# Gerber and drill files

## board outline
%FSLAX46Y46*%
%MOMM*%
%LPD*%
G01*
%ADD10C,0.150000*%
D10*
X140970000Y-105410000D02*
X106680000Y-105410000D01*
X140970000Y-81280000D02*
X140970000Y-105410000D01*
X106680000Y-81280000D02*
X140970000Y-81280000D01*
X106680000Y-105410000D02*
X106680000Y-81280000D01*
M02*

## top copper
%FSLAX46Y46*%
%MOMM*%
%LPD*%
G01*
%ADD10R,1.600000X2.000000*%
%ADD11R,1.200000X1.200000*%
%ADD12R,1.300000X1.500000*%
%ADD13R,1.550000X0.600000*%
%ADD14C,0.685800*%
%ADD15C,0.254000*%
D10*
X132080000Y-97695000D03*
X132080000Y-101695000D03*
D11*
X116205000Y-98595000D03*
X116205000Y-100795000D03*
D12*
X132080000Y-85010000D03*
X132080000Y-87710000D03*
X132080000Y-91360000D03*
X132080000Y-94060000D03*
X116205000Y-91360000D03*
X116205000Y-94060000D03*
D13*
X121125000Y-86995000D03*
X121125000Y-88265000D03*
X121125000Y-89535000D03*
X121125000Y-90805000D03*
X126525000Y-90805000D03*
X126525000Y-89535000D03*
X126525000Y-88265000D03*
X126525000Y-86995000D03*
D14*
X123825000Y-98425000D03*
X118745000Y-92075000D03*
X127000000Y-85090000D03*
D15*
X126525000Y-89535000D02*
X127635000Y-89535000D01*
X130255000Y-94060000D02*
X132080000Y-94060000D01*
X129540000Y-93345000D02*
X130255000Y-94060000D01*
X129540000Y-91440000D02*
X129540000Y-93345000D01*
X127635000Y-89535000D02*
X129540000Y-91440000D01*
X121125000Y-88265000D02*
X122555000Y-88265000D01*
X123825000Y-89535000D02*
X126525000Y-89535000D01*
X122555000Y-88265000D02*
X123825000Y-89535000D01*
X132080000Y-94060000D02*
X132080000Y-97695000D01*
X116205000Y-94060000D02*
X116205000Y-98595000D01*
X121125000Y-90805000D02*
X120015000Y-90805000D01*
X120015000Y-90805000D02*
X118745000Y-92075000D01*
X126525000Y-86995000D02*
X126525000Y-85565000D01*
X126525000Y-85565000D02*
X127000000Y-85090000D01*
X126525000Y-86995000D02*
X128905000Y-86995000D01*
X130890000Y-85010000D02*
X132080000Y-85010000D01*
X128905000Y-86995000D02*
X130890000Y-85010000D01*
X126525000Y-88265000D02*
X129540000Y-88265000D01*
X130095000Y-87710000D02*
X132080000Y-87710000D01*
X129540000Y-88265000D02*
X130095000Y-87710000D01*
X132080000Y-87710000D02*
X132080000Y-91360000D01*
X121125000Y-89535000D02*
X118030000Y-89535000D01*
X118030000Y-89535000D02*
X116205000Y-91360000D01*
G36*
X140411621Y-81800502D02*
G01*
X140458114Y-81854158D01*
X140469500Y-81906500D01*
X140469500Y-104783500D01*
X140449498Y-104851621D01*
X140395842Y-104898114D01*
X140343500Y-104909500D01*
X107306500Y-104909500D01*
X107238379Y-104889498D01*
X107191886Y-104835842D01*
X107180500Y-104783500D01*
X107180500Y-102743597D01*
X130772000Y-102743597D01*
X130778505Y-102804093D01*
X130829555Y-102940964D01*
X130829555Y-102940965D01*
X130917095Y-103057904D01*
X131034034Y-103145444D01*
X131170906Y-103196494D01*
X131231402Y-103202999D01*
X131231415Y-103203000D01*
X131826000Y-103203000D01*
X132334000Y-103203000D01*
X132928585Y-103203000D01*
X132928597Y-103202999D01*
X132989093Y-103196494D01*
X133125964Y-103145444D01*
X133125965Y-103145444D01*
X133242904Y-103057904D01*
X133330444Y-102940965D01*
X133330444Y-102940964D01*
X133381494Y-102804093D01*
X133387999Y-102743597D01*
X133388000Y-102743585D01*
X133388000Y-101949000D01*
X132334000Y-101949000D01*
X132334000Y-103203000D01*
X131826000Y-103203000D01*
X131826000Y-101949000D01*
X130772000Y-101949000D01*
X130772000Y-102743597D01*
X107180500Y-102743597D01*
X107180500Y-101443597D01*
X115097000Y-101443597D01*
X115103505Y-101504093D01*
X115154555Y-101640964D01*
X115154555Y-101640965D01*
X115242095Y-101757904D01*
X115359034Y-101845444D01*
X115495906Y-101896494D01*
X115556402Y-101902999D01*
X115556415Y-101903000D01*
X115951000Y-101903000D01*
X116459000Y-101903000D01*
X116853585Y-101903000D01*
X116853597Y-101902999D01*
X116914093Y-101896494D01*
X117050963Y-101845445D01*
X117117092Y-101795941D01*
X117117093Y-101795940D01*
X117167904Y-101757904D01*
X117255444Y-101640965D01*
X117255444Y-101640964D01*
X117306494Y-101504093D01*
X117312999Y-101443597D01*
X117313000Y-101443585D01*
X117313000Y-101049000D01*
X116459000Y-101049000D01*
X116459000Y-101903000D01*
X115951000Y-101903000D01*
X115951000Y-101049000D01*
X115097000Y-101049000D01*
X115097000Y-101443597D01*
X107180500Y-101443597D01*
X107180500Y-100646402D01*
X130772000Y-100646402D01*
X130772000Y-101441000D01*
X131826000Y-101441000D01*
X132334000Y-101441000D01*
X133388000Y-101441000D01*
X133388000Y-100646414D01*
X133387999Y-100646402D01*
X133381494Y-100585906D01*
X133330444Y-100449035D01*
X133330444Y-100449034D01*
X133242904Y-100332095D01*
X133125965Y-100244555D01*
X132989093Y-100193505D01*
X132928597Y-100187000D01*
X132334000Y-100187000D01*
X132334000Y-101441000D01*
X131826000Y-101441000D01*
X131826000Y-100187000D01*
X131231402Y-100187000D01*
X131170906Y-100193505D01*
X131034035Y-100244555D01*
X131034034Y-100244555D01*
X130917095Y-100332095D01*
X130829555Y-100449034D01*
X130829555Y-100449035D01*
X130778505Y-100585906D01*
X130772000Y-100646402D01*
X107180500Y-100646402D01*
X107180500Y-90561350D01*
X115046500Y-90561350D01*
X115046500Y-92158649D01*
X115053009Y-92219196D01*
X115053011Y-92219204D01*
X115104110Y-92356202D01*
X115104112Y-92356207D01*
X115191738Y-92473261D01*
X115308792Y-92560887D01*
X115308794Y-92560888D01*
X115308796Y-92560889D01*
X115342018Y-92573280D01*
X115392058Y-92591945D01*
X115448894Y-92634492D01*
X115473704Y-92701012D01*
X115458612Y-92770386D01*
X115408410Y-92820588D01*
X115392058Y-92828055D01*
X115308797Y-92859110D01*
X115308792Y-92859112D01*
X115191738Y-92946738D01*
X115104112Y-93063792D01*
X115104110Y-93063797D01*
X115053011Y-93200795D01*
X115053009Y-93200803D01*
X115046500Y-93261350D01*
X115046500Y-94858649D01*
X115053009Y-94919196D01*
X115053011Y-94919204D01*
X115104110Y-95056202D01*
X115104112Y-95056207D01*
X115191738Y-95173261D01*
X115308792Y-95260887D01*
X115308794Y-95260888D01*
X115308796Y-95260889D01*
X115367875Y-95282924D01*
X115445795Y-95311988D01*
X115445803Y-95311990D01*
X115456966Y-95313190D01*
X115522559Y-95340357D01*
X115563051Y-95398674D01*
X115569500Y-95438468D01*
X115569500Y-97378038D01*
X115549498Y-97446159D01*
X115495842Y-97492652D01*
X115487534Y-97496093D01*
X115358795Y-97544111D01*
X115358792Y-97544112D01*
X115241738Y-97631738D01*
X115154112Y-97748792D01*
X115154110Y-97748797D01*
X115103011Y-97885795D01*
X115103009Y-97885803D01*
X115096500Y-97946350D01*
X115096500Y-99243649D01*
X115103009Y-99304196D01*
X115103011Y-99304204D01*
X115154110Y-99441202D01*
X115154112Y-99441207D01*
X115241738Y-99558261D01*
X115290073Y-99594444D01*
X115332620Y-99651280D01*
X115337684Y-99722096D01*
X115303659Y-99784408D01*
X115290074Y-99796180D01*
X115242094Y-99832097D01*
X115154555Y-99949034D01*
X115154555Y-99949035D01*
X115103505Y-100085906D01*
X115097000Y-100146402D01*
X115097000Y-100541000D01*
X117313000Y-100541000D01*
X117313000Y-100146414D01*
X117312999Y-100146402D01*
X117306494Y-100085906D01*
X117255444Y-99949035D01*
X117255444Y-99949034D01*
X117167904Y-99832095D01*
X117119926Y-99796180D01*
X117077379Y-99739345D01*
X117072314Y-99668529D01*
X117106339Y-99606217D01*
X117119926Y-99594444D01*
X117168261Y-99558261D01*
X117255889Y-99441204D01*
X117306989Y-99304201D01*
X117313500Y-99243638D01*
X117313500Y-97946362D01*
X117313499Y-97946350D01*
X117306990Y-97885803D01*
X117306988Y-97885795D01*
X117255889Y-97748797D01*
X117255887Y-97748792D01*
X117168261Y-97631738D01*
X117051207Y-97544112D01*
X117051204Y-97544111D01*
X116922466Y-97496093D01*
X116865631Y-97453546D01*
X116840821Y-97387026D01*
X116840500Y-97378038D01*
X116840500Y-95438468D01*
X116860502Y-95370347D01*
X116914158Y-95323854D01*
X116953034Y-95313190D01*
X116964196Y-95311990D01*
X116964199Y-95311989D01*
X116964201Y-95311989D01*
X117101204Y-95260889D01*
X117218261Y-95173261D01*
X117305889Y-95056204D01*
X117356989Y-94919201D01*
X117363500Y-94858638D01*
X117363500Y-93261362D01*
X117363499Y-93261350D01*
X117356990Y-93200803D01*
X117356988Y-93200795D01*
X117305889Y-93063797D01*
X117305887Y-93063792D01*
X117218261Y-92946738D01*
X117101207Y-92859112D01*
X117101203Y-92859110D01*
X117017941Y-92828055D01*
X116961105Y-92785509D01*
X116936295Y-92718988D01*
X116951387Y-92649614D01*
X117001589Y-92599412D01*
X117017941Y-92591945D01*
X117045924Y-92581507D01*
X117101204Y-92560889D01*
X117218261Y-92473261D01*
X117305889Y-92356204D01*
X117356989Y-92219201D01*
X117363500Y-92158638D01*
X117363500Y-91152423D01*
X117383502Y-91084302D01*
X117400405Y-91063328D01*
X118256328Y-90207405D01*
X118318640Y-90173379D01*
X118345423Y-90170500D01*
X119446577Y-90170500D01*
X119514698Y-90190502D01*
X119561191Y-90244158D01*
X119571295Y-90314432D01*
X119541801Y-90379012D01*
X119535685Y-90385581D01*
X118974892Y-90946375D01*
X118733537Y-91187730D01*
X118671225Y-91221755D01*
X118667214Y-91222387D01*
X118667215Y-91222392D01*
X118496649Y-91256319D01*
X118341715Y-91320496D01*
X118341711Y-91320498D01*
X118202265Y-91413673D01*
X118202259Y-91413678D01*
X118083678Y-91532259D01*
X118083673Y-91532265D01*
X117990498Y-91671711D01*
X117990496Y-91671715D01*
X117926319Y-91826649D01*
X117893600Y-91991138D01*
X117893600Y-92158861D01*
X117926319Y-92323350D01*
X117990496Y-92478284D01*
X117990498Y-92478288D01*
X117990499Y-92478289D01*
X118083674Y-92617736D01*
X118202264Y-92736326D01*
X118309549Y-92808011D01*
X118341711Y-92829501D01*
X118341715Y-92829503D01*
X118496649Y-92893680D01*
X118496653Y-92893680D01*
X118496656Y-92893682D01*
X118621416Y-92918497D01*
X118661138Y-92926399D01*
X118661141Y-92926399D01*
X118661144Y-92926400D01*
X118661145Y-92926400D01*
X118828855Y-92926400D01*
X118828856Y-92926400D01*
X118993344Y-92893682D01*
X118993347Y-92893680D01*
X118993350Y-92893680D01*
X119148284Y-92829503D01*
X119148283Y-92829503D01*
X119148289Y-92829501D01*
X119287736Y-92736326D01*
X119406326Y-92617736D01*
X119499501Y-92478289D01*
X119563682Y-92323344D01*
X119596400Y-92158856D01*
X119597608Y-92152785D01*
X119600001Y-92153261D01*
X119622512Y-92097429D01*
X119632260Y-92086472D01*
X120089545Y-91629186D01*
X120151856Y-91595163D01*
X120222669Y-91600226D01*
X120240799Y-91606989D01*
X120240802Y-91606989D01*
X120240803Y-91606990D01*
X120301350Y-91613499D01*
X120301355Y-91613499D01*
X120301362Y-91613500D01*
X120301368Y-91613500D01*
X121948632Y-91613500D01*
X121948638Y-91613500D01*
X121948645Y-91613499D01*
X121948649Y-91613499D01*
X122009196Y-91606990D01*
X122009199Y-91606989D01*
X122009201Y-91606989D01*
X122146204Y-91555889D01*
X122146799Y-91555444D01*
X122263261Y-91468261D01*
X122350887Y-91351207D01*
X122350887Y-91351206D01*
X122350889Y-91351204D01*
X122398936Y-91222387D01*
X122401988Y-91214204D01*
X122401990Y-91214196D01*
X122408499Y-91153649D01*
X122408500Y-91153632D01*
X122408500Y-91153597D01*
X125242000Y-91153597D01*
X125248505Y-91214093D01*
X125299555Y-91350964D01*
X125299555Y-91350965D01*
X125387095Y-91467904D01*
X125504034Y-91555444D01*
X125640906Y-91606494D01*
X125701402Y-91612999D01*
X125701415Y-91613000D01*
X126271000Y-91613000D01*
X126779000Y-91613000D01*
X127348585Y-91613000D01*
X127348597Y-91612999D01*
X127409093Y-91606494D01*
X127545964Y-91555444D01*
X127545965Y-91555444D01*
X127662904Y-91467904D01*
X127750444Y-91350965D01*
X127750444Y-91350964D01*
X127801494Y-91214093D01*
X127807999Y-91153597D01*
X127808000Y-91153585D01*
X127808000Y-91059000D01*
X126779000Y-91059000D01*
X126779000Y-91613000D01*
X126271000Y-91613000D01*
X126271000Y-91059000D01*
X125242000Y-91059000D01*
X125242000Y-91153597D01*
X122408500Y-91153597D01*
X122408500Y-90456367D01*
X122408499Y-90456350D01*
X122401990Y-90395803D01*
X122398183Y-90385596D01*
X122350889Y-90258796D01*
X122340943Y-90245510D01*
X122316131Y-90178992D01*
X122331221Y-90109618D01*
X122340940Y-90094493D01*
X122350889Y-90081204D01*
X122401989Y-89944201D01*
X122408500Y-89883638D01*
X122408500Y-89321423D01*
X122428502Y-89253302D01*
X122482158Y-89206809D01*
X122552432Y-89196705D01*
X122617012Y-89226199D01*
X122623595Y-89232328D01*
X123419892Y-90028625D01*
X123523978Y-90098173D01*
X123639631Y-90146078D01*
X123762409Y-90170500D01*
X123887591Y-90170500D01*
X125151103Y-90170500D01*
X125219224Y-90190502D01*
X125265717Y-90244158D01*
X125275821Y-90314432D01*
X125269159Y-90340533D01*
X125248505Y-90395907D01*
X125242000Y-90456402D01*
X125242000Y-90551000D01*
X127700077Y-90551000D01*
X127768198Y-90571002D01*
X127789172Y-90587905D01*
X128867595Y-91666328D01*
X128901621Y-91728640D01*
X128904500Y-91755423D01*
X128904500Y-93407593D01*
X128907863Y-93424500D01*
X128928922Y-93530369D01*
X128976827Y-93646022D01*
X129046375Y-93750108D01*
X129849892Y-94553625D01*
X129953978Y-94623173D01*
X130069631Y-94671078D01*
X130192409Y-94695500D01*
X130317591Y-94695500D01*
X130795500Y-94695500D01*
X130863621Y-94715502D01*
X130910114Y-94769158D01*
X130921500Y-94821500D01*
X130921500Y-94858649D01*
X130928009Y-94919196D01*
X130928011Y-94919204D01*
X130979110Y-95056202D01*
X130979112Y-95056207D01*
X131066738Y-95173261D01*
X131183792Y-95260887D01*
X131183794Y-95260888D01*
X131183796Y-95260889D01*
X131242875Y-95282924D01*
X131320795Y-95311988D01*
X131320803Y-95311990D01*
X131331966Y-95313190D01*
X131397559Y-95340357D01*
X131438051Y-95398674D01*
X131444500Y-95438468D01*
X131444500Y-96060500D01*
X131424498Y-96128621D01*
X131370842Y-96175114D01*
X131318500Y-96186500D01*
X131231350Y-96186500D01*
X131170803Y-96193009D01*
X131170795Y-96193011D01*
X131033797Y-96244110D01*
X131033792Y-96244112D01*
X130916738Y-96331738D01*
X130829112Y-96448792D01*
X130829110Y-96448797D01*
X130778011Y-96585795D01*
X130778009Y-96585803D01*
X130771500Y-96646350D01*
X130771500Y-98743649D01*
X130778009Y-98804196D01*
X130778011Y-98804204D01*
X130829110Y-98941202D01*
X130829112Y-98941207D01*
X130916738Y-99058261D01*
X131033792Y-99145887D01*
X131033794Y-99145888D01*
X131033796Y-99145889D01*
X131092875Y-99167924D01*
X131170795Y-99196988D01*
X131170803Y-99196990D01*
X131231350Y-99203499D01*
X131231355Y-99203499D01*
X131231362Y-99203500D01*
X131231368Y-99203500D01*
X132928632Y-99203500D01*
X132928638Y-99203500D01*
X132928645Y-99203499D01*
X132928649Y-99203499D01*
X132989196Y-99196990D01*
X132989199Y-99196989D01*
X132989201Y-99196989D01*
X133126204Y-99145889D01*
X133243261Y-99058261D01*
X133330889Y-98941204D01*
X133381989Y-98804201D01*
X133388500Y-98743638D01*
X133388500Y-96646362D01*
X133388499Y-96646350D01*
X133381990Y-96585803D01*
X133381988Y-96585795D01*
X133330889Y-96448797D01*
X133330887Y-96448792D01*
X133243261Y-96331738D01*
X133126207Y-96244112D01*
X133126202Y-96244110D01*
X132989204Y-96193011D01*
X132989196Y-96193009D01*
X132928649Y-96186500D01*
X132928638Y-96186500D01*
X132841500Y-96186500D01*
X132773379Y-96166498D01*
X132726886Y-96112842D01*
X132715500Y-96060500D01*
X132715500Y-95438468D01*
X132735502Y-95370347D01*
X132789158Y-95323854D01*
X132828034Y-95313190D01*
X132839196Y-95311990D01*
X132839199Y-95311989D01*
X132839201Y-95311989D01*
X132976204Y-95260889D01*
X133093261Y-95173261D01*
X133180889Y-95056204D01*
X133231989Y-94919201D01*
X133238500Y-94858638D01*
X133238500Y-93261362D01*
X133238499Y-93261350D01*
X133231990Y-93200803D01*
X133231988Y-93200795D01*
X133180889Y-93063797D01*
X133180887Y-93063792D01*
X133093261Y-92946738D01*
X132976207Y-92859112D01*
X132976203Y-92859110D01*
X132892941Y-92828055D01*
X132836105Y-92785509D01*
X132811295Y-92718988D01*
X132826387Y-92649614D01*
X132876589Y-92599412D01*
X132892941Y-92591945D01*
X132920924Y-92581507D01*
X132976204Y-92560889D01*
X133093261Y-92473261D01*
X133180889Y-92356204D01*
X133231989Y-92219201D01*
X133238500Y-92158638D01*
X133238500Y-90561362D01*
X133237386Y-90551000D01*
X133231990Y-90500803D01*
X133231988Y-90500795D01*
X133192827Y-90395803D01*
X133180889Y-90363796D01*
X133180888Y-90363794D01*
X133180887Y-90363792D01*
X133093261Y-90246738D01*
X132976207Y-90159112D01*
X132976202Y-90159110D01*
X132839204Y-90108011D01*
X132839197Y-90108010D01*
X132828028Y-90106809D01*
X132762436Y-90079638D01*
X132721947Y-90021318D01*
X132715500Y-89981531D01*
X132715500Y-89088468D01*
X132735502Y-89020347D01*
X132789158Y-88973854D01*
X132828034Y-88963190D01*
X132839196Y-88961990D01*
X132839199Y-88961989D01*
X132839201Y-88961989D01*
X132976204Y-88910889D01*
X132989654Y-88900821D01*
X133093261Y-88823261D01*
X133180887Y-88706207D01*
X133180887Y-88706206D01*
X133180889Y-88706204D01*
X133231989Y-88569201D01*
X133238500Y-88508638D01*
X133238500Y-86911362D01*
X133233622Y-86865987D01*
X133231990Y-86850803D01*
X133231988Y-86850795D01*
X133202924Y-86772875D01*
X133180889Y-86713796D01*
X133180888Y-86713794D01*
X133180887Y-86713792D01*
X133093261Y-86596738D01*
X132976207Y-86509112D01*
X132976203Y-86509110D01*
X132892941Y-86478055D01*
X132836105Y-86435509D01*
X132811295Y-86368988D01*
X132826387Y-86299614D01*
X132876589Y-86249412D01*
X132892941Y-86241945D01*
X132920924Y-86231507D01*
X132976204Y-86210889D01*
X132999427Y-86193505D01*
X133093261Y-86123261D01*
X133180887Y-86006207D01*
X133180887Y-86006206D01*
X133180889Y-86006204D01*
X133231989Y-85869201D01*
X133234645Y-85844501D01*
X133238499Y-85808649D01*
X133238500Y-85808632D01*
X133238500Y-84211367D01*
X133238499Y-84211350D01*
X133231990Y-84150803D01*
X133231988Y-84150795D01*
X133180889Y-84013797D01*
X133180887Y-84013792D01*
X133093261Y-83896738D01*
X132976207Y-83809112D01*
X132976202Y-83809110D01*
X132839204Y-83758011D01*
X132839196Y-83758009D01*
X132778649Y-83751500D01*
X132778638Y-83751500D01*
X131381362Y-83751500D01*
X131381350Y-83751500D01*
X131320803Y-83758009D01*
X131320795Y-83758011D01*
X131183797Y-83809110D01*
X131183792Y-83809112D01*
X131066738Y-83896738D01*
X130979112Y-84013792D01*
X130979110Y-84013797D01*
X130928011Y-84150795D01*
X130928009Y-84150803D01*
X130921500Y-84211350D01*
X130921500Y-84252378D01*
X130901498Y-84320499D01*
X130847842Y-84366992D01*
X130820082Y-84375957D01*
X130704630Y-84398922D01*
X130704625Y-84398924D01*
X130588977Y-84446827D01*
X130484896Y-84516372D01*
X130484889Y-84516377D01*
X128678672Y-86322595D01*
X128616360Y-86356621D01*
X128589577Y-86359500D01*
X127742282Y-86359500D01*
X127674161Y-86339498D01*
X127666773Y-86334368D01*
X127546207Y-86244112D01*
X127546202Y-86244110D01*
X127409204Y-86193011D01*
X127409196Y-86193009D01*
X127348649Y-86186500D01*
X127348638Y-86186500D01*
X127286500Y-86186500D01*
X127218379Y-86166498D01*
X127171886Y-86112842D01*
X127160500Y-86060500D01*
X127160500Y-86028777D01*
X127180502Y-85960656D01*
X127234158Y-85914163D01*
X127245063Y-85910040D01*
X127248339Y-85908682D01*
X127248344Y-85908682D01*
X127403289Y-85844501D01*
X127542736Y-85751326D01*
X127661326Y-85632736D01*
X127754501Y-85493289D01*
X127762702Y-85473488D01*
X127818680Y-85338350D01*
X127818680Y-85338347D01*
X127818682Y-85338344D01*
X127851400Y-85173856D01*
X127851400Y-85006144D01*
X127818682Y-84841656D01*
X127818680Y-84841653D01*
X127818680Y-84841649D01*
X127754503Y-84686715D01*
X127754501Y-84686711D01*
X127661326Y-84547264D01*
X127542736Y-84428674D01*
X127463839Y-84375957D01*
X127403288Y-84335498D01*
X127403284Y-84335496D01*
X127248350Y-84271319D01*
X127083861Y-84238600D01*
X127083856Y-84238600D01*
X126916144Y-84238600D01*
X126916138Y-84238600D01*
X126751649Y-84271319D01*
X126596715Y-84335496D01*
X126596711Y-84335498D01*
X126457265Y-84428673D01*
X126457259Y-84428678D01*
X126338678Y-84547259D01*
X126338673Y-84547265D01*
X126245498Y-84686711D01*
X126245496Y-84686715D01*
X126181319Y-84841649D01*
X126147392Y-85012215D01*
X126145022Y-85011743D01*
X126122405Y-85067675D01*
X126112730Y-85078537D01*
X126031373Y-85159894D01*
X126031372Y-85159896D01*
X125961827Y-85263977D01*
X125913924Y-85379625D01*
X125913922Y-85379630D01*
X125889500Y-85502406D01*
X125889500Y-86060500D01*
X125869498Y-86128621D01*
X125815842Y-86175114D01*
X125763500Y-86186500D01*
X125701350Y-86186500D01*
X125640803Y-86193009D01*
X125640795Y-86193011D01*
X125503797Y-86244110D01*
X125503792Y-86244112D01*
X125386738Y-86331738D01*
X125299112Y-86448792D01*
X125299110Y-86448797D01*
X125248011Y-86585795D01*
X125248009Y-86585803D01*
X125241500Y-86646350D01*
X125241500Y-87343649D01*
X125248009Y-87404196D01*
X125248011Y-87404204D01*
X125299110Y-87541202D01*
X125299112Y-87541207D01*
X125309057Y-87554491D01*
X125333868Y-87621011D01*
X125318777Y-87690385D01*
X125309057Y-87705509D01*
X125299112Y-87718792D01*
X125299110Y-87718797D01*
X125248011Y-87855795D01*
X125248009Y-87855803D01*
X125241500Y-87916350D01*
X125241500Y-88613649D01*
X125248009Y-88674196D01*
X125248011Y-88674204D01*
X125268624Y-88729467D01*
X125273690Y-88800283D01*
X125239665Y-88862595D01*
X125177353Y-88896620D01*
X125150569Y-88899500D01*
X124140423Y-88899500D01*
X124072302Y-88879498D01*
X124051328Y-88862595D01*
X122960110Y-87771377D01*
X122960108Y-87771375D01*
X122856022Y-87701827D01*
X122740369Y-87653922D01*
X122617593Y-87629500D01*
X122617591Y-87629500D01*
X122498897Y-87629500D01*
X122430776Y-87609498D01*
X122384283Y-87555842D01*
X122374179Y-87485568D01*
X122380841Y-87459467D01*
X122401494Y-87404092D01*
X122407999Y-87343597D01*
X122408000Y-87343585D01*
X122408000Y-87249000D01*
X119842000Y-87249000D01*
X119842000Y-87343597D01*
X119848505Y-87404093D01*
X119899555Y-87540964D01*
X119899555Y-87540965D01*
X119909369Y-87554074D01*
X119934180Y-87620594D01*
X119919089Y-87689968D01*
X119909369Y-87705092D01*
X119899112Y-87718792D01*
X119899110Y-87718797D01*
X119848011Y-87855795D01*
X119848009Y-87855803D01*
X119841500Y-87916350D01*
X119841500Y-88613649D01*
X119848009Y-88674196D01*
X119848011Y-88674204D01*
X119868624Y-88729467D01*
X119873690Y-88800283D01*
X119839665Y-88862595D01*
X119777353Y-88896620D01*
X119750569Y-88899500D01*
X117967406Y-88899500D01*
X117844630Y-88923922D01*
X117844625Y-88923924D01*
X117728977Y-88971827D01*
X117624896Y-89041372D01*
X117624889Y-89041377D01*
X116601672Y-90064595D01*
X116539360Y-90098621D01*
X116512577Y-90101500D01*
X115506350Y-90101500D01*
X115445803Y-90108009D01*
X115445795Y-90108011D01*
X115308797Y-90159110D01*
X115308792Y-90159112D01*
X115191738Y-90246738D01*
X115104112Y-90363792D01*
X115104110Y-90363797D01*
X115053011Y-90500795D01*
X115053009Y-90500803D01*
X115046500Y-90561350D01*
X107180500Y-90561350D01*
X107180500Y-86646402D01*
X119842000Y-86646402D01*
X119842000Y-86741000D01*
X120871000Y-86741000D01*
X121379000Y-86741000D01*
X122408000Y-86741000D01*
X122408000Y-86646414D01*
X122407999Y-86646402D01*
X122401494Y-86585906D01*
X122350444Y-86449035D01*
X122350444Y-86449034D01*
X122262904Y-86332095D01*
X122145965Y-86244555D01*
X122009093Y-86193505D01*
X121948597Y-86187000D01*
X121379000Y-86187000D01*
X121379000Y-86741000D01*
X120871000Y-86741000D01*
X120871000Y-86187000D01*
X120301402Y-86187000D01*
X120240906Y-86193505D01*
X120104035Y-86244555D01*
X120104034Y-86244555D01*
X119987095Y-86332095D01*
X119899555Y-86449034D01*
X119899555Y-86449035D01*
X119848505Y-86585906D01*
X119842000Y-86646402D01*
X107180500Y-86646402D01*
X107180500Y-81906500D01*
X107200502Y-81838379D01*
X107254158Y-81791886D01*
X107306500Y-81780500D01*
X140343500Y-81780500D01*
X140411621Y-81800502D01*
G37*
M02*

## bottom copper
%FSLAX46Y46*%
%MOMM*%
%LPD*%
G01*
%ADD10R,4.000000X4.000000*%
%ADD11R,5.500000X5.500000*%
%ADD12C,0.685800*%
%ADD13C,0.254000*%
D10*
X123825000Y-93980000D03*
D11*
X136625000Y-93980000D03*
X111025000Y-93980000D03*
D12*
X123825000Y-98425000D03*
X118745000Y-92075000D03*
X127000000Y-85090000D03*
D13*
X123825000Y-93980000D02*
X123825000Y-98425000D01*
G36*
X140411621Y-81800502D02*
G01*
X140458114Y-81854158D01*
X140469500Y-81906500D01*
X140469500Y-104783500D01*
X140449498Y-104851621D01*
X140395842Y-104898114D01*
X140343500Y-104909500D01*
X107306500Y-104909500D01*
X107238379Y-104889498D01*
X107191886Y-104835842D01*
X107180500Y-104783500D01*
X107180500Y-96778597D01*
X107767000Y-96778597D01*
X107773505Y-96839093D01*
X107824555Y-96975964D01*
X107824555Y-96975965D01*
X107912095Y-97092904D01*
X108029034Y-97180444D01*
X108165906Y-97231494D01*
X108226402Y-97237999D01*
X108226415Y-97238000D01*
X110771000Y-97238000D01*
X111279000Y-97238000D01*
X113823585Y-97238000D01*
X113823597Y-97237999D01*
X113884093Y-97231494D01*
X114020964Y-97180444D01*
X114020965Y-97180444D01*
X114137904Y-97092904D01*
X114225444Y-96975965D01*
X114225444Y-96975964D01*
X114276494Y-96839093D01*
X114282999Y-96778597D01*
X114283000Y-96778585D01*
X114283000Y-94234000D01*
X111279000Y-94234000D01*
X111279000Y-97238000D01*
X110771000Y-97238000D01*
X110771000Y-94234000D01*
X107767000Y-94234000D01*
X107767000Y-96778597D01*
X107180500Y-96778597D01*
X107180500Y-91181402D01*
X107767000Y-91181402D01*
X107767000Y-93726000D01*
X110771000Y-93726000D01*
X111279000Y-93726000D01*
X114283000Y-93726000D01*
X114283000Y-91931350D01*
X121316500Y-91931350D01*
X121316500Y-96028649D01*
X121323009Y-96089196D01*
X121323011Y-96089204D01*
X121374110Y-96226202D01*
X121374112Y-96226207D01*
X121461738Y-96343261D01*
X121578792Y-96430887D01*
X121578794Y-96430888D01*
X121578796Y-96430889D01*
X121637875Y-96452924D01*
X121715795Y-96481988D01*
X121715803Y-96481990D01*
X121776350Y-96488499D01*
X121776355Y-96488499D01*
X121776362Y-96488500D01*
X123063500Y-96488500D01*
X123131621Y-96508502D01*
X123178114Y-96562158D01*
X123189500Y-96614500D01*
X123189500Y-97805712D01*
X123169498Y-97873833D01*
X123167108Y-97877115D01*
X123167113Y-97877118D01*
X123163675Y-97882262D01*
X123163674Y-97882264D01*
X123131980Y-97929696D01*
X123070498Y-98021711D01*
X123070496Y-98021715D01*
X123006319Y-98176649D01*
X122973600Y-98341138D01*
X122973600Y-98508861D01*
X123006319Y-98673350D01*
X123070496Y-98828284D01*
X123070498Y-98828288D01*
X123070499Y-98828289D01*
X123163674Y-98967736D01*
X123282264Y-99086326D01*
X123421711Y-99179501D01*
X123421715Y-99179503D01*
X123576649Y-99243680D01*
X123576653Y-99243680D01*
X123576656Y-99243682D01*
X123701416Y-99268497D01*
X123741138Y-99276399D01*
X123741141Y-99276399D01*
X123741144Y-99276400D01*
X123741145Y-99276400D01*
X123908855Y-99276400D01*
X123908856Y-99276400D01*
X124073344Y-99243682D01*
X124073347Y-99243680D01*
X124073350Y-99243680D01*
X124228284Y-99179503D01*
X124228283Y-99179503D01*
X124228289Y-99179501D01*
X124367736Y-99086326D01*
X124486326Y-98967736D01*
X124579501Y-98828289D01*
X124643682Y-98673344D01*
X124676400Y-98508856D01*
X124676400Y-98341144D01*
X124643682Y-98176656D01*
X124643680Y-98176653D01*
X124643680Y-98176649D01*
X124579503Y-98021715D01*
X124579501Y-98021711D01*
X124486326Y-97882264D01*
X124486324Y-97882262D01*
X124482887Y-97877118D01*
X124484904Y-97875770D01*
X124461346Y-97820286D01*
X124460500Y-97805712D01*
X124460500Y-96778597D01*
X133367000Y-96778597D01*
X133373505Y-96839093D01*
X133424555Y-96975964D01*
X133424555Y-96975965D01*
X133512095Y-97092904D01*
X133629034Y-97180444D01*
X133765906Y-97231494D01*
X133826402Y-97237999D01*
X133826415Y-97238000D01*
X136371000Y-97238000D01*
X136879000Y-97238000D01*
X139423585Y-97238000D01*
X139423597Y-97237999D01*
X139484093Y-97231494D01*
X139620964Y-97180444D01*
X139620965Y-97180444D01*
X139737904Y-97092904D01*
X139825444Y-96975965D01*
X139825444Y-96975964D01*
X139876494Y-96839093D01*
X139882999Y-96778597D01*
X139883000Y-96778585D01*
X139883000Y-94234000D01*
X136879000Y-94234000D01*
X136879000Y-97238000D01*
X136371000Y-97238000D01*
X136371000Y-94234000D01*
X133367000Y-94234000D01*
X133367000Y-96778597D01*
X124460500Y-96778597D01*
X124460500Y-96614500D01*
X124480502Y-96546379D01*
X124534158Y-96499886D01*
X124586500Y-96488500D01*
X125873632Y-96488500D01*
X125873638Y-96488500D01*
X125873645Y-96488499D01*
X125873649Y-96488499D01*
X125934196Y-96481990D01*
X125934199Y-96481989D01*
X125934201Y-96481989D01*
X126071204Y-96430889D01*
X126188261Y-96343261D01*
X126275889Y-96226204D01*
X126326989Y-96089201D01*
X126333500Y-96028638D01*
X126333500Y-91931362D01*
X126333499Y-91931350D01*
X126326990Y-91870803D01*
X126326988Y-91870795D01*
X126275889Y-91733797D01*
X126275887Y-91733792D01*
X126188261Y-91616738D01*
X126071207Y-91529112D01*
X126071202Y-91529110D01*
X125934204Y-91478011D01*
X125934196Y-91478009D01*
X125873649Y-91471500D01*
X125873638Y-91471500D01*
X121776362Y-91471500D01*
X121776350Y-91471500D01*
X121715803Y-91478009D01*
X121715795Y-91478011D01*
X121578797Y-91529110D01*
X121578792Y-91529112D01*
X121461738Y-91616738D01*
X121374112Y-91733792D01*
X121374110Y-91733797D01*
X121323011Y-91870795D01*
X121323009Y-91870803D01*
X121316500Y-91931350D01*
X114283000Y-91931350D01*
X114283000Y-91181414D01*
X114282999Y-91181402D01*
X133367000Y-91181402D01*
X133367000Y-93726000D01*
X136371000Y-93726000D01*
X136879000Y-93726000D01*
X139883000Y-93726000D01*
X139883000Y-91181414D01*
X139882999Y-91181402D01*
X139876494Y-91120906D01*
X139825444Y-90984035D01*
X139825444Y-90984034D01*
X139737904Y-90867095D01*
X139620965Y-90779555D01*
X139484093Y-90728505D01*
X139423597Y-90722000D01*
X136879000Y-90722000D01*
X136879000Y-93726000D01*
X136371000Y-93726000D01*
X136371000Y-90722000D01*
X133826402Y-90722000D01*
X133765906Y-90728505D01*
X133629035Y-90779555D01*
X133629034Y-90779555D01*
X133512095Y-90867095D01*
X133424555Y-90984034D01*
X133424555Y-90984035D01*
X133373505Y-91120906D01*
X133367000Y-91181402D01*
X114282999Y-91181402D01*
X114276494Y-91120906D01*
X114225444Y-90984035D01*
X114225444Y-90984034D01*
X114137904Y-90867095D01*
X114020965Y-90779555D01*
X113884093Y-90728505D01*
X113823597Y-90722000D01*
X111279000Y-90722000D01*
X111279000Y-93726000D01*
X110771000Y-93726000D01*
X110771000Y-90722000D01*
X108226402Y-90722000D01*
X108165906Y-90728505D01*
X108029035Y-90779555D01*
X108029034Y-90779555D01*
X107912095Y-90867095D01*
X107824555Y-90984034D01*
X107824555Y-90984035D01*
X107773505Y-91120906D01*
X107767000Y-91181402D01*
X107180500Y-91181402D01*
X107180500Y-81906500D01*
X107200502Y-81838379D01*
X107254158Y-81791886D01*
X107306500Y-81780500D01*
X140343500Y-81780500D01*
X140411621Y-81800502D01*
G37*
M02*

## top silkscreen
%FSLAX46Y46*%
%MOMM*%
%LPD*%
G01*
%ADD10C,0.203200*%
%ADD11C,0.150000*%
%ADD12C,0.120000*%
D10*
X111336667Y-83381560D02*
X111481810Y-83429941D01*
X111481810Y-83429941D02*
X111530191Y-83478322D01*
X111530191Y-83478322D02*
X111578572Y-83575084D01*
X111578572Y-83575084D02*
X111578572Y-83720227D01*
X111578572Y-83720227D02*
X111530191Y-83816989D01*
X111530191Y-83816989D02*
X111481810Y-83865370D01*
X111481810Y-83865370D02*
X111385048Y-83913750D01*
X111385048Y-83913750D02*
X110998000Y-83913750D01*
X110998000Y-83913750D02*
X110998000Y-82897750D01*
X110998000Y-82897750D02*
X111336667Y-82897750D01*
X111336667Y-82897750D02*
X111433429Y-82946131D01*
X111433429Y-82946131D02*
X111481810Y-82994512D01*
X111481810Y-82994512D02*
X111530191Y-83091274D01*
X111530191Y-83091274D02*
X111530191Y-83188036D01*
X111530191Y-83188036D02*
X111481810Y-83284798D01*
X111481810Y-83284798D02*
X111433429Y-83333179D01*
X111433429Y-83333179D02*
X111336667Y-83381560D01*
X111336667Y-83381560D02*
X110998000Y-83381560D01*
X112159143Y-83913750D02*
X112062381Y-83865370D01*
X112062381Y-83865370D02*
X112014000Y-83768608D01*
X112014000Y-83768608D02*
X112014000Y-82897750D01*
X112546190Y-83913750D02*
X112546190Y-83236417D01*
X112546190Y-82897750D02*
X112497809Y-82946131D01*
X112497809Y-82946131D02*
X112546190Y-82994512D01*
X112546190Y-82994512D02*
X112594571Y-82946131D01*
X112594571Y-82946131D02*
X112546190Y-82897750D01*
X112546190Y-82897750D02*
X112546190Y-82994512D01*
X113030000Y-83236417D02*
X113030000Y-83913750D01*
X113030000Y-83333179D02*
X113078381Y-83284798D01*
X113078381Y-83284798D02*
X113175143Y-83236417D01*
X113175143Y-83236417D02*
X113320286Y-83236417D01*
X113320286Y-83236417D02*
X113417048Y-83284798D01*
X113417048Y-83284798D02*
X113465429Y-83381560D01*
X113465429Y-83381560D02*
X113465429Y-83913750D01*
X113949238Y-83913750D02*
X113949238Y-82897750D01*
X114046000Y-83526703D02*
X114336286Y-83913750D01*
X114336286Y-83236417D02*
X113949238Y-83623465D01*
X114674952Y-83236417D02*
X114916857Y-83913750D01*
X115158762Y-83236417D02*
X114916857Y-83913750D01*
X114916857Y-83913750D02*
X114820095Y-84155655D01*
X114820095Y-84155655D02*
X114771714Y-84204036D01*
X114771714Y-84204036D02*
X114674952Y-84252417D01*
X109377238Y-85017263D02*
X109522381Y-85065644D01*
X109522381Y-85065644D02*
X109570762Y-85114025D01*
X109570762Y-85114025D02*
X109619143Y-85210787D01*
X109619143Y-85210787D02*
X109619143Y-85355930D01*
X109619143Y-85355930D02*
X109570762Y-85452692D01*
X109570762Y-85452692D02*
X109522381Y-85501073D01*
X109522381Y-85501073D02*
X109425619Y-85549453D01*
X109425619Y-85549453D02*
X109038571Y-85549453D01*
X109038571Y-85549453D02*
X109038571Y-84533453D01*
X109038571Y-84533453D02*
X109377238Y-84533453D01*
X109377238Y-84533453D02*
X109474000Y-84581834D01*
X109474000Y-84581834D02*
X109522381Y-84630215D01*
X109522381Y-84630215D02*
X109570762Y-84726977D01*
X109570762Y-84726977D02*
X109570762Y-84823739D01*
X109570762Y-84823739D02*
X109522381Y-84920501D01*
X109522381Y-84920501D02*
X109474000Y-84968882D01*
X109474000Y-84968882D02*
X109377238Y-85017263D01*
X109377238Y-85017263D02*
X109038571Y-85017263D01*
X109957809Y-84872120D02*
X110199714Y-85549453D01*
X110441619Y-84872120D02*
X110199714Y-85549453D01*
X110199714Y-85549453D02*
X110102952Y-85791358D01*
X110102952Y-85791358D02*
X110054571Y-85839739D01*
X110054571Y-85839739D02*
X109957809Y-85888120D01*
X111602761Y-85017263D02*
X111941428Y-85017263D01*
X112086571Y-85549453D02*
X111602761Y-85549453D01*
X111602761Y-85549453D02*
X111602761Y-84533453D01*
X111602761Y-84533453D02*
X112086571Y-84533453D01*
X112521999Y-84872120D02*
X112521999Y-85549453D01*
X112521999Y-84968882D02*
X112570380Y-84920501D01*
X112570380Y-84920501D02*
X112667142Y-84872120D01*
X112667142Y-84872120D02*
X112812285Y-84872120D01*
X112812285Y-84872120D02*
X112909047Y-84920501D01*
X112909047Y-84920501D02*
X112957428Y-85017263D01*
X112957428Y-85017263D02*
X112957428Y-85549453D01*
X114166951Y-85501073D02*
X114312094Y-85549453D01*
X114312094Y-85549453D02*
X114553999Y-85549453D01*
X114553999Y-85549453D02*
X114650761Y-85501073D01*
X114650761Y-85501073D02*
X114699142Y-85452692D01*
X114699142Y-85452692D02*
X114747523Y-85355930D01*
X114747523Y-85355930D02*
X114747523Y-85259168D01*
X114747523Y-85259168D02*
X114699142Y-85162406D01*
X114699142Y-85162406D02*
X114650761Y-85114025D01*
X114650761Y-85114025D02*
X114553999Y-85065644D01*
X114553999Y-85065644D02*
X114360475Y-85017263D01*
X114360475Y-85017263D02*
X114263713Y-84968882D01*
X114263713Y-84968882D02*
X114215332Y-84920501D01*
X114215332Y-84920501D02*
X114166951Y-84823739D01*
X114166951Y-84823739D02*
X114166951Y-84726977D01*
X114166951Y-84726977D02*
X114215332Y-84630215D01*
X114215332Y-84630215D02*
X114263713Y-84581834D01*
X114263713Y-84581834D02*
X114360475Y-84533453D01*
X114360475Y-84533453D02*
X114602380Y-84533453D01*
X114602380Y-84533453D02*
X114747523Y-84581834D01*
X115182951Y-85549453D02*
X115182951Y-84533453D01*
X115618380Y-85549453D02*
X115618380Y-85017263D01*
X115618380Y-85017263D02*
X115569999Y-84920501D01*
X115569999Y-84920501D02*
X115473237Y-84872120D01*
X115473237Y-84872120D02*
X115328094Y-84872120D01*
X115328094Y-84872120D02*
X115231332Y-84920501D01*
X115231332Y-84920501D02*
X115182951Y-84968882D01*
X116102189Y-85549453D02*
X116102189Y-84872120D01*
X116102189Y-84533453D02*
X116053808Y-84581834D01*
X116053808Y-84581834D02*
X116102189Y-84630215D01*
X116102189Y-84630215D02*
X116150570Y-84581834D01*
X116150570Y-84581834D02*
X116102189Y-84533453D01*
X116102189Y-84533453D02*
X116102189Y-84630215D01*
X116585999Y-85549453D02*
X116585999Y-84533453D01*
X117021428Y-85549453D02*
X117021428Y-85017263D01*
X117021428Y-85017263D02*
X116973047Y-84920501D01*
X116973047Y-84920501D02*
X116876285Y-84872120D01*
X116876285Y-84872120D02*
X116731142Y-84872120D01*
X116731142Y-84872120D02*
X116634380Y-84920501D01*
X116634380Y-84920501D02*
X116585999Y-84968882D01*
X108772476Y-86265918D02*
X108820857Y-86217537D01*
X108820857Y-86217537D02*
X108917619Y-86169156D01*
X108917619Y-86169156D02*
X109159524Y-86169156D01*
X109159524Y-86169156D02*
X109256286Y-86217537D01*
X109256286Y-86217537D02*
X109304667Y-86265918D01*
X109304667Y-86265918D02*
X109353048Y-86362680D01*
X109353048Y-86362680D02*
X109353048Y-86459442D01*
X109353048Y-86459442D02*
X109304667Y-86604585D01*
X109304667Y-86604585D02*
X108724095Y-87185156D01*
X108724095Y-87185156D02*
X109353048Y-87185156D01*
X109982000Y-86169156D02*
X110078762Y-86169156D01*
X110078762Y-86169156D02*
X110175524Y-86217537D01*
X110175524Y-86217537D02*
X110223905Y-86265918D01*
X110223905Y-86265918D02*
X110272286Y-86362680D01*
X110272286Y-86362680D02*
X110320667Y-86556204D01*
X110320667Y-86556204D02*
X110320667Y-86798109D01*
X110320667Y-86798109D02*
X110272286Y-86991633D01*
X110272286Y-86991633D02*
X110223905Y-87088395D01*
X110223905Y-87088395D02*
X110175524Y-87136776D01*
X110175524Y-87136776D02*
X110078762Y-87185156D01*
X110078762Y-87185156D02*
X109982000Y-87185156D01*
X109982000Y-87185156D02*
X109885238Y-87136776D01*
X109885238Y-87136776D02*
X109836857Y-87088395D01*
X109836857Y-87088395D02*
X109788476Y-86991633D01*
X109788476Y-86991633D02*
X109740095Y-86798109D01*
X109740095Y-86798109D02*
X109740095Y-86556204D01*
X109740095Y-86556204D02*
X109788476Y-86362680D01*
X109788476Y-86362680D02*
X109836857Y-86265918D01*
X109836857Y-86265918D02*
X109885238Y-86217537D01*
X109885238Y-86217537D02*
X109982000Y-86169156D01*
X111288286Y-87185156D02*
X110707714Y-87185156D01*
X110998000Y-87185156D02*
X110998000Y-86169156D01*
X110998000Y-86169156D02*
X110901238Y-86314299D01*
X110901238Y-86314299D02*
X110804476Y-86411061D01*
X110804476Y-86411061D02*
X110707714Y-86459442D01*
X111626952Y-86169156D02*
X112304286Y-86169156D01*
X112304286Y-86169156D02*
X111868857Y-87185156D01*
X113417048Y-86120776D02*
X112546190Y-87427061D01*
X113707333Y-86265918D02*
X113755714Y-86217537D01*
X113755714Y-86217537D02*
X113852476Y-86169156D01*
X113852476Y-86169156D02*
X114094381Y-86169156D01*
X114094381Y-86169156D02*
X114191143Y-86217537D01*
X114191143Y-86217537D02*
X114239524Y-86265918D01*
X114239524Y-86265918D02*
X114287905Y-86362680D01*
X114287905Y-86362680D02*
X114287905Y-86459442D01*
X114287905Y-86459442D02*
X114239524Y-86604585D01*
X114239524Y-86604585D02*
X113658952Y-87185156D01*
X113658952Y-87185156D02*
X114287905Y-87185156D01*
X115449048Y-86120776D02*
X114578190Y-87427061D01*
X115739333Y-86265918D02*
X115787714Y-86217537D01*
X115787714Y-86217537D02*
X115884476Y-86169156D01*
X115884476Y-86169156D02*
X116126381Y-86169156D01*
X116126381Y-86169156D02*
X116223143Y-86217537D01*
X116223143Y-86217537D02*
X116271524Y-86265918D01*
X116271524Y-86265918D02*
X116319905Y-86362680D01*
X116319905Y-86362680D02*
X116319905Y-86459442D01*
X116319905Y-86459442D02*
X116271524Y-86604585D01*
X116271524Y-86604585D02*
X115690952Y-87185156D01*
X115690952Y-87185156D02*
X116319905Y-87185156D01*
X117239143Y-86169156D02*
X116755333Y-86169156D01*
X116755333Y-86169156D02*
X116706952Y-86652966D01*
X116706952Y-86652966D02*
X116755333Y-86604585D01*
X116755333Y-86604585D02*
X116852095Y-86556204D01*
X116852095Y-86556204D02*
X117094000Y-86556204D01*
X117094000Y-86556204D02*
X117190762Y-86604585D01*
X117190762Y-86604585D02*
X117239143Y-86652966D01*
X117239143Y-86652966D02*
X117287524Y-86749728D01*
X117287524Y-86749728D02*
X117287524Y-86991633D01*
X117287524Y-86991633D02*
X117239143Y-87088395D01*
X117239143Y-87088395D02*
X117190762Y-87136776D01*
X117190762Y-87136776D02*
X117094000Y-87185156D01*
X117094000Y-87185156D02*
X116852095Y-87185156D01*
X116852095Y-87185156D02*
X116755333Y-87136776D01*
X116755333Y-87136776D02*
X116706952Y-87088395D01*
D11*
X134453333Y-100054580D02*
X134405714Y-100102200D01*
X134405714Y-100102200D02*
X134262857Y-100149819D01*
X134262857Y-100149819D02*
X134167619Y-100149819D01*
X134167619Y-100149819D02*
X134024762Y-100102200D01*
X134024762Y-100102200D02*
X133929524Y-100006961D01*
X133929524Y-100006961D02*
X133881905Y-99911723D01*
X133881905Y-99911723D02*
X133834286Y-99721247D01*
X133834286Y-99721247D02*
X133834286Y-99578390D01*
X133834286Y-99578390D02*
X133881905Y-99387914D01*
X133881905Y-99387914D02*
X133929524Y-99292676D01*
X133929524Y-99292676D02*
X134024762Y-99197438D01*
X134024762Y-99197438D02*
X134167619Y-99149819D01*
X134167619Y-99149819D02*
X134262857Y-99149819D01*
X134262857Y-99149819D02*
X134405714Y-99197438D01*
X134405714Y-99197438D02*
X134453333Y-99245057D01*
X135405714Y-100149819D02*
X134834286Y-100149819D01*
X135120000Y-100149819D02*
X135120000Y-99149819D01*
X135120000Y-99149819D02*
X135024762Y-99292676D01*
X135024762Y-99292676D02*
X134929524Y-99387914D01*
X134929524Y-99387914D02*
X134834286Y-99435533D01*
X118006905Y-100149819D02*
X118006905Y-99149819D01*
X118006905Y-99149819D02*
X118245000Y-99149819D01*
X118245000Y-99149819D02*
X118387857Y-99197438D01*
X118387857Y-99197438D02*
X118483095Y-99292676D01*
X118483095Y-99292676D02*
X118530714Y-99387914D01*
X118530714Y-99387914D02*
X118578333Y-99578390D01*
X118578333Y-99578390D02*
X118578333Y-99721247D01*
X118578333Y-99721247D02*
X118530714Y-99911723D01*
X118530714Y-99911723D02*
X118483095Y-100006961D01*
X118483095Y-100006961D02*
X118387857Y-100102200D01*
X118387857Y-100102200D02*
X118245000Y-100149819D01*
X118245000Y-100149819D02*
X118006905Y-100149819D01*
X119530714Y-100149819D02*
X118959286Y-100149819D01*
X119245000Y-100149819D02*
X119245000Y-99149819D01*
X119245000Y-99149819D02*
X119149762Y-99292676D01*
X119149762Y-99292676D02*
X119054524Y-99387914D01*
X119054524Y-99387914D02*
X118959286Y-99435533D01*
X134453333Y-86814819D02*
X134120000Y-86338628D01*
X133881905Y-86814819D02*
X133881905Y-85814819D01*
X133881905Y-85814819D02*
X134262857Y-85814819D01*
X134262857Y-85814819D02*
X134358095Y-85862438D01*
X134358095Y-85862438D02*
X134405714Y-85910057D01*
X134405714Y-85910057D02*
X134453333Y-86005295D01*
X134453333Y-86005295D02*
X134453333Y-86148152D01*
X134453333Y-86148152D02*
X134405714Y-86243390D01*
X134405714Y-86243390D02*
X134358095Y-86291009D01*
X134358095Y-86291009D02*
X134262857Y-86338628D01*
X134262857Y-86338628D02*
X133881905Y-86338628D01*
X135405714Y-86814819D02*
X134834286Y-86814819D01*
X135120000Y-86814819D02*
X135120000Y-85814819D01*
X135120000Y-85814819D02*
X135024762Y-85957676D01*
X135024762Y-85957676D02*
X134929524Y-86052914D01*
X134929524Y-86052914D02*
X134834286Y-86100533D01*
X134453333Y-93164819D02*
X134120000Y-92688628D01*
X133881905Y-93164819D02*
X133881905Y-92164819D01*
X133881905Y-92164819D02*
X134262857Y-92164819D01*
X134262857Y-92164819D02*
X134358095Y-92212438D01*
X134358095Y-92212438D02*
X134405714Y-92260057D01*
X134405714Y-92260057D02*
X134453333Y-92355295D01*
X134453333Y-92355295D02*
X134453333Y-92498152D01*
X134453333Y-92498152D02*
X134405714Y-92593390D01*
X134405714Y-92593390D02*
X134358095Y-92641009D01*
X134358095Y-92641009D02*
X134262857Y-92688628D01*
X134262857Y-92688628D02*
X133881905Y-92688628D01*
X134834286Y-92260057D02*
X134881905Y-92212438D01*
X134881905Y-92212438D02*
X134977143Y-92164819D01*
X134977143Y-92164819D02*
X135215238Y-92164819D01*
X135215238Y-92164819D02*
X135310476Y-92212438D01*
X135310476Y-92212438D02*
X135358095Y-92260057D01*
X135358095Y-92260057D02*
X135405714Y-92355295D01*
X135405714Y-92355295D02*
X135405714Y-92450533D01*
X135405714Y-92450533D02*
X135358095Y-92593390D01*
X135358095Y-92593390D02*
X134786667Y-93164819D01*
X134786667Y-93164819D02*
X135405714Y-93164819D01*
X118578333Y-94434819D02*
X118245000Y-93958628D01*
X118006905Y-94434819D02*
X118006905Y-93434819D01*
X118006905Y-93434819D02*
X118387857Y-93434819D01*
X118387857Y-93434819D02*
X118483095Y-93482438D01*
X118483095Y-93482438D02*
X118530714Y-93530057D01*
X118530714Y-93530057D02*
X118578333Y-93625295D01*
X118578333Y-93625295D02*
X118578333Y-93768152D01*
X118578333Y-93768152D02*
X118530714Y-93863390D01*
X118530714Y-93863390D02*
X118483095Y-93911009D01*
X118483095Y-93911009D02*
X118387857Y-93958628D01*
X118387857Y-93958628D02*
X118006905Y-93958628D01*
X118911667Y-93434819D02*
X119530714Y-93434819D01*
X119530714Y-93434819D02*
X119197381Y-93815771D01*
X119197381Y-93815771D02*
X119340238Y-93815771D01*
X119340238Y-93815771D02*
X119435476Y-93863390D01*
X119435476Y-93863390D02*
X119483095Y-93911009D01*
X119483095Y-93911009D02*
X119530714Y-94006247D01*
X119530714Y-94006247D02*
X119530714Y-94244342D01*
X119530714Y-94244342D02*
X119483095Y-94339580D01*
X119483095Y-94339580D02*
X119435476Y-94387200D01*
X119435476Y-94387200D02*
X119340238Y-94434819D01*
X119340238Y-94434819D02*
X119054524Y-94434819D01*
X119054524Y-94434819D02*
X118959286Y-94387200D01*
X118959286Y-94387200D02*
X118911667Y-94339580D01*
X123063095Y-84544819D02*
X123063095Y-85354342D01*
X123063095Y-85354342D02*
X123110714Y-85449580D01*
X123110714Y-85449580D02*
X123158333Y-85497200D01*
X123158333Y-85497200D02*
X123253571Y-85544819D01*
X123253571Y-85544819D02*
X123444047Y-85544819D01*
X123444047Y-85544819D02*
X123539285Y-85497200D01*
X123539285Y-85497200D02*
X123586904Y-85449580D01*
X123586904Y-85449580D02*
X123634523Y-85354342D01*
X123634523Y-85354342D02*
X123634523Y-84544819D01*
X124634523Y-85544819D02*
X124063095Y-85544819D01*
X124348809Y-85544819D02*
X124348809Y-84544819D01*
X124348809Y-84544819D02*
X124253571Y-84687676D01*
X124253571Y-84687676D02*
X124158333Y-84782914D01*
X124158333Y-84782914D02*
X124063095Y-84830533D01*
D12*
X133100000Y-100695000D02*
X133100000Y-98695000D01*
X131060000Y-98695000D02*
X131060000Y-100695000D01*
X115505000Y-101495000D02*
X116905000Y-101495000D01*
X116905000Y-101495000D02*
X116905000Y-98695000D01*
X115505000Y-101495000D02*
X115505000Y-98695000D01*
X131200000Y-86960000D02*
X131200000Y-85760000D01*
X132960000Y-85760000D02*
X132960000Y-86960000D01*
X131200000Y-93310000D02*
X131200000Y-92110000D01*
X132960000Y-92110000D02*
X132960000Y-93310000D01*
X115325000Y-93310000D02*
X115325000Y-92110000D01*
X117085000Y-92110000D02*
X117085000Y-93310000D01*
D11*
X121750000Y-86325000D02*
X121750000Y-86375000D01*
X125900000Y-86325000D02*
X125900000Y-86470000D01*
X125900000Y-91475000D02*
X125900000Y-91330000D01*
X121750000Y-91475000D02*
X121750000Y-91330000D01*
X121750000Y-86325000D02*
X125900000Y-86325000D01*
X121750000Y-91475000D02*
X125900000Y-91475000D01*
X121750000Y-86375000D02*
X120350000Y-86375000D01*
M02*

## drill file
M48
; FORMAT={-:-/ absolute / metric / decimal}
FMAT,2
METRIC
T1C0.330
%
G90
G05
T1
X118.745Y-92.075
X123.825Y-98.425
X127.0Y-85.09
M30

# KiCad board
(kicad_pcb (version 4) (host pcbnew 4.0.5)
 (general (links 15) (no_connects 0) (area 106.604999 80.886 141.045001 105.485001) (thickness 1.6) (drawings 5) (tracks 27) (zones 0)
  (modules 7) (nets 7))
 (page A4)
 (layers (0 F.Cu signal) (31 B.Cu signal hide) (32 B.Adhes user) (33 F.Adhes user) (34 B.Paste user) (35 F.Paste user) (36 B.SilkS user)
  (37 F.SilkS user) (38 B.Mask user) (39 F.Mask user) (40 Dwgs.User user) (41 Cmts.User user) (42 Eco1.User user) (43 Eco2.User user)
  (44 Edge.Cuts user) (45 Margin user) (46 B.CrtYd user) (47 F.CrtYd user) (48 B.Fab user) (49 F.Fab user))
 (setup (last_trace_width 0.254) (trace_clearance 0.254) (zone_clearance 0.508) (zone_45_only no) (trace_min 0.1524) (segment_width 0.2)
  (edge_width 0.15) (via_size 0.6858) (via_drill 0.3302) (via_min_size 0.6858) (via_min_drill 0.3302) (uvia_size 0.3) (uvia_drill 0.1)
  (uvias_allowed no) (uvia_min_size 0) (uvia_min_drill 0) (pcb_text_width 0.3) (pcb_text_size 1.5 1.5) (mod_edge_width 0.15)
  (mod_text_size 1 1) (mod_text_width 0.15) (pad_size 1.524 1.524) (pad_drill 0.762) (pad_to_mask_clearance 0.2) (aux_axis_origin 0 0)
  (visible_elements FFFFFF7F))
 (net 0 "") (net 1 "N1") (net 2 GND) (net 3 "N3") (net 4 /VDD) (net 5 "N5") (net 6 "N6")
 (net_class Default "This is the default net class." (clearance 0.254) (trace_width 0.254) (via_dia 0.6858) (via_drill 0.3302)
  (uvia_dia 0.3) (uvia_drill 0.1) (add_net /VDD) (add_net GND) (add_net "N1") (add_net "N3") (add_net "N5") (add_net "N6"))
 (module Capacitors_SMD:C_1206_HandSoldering (layer F.Cu) (at 132.08 99.695 270)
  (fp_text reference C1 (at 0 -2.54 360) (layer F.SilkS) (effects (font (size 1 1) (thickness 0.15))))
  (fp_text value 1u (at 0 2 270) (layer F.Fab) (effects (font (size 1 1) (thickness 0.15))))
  (fp_line (start 1 -1.02) (end -1 -1.02) (layer F.SilkS) (width 0.12))
  (fp_line (start -1 1.02) (end 1 1.02) (layer F.SilkS) (width 0.12))
  (pad 1 smd rect (at -2 0 270) (size 2 1.6) (layers F.Cu F.Paste F.Mask) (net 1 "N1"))
  (pad 2 smd rect (at 2 0 270) (size 2 1.6) (layers F.Cu F.Paste F.Mask) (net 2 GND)))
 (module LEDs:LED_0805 (layer F.Cu) (at 116.205 99.695 90)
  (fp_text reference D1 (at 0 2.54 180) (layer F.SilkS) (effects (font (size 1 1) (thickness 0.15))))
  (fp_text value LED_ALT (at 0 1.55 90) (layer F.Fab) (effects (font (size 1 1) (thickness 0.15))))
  (fp_line (start -1.8 -0.7) (end -1.8 0.7) (layer F.SilkS) (width 0.12))
  (fp_line (start -1.8 0.7) (end 1 0.7) (layer F.SilkS) (width 0.12))
  (fp_line (start -1.8 -0.7) (end 1 -0.7) (layer F.SilkS) (width 0.12))
  (pad 2 smd rect (at 1.1 0 270) (size 1.2 1.2) (layers F.Cu F.Paste F.Mask) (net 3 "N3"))
  (pad 1 smd rect (at -1.1 0 270) (size 1.2 1.2) (layers F.Cu F.Paste F.Mask) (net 2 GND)))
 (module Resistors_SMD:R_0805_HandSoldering (layer F.Cu) (at 132.08 86.36 270)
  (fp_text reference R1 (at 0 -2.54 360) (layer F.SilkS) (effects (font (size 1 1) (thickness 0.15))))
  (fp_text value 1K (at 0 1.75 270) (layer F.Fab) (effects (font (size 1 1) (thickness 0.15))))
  (fp_line (start 0.6 0.88) (end -0.6 0.88) (layer F.SilkS) (width 0.12))
  (fp_line (start -0.6 -0.88) (end 0.6 -0.88) (layer F.SilkS) (width 0.12))
  (pad 1 smd rect (at -1.35 0 270) (size 1.5 1.3) (layers F.Cu F.Paste F.Mask) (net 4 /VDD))
  (pad 2 smd rect (at 1.35 0 270) (size 1.5 1.3) (layers F.Cu F.Paste F.Mask) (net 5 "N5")))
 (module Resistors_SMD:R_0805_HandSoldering (layer F.Cu) (at 132.08 92.71 270)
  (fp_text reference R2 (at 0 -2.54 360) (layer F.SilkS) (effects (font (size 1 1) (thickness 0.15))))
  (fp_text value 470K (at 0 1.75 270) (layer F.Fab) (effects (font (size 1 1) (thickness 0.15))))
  (fp_line (start 0.6 0.88) (end -0.6 0.88) (layer F.SilkS) (width 0.12))
  (fp_line (start -0.6 -0.88) (end 0.6 -0.88) (layer F.SilkS) (width 0.12))
  (pad 1 smd rect (at -1.35 0 270) (size 1.5 1.3) (layers F.Cu F.Paste F.Mask) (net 5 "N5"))
  (pad 2 smd rect (at 1.35 0 270) (size 1.5 1.3) (layers F.Cu F.Paste F.Mask) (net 1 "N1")))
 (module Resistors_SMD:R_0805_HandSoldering (layer F.Cu) (at 116.205 92.71 270)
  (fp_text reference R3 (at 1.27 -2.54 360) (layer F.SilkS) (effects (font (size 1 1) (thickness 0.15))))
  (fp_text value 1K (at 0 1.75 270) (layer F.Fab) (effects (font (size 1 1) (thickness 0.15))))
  (fp_line (start 0.6 0.88) (end -0.6 0.88) (layer F.SilkS) (width 0.12))
  (fp_line (start -0.6 -0.88) (end 0.6 -0.88) (layer F.SilkS) (width 0.12))
  (pad 1 smd rect (at -1.35 0 270) (size 1.5 1.3) (layers F.Cu F.Paste F.Mask) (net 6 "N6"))
  (pad 2 smd rect (at 1.35 0 270) (size 1.5 1.3) (layers F.Cu F.Paste F.Mask) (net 3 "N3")))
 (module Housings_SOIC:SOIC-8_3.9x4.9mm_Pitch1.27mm (layer F.Cu) (at 123.825 88.9)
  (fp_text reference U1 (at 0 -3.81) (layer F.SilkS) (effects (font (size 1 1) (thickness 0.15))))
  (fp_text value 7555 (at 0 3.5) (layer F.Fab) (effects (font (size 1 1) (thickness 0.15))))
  (fp_line (start -2.075 -2.575) (end -2.075 -2.525) (layer F.SilkS) (width 0.15))
  (fp_line (start 2.075 -2.575) (end 2.075 -2.43) (layer F.SilkS) (width 0.15))
  (fp_line (start 2.075 2.575) (end 2.075 2.43) (layer F.SilkS) (width 0.15))
  (fp_line (start -2.075 2.575) (end -2.075 2.43) (layer F.SilkS) (width 0.15))
  (fp_line (start -2.075 -2.575) (end 2.075 -2.575) (layer F.SilkS) (width 0.15))
  (fp_line (start -2.075 2.575) (end 2.075 2.575) (layer F.SilkS) (width 0.15))
  (fp_line (start -2.075 -2.525) (end -3.475 -2.525) (layer F.SilkS) (width 0.15))
  (pad 1 smd rect (at -2.7 -1.905) (size 1.55 0.6) (layers F.Cu F.Paste F.Mask) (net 2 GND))
  (pad 2 smd rect (at -2.7 -0.635) (size 1.55 0.6) (layers F.Cu F.Paste F.Mask) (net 1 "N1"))
  (pad 3 smd rect (at -2.7 0.635) (size 1.55 0.6) (layers F.Cu F.Paste F.Mask) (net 6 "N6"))
  (pad 4 smd rect (at -2.7 1.905) (size 1.55 0.6) (layers F.Cu F.Paste F.Mask) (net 4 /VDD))
  (pad 5 smd rect (at 2.7 1.905) (size 1.55 0.6) (layers F.Cu F.Paste F.Mask) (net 2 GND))
  (pad 6 smd rect (at 2.7 0.635) (size 1.55 0.6) (layers F.Cu F.Paste F.Mask) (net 1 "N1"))
  (pad 7 smd rect (at 2.7 -0.635) (size 1.55 0.6) (layers F.Cu F.Paste F.Mask) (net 5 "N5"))
  (pad 8 smd rect (at 2.7 -1.905) (size 1.55 0.6) (layers F.Cu F.Paste F.Mask) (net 4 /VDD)))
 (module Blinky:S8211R (layer B.Cu) (at 123.825 93.98 180)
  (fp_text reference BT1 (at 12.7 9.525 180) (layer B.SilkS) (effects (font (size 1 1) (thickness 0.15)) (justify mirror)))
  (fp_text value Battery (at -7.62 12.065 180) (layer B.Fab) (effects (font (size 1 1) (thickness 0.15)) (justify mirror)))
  (pad 2 smd rect (at 0 0 180) (size 4 4) (layers B.Cu B.Paste B.Mask) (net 2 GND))
  (pad 1 smd rect (at -12.8 0 180) (size 5.5 5.5) (layers B.Cu B.Paste B.Mask) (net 4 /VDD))
  (pad 1 smd rect (at 12.8 0 180) (size 5.5 5.5) (layers B.Cu B.Paste B.Mask) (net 4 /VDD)))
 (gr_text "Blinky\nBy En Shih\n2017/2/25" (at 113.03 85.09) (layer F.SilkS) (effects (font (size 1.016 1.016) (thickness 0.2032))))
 (gr_line (start 140.97 105.41) (end 106.68 105.41) (angle 90) (layer Edge.Cuts) (width 0.15))
 (gr_line (start 140.97 81.28) (end 140.97 105.41) (angle 90) (layer Edge.Cuts) (width 0.15))
 (gr_line (start 106.68 81.28) (end 140.97 81.28) (angle 90) (layer Edge.Cuts) (width 0.15))
 (gr_line (start 106.68 105.41) (end 106.68 81.28) (angle 90) (layer Edge.Cuts) (width 0.15))
 (segment (start 126.525 89.535) (end 127.635 89.535) (width 0.254) (layer F.Cu) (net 1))
 (segment (start 130.255 94.06) (end 132.08 94.06) (width 0.254) (layer F.Cu) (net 1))
 (segment (start 129.54 93.345) (end 130.255 94.06) (width 0.254) (layer F.Cu) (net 1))
 (segment (start 129.54 91.44) (end 129.54 93.345) (width 0.254) (layer F.Cu) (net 1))
 (segment (start 127.635 89.535) (end 129.54 91.44) (width 0.254) (layer F.Cu) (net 1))
 (segment (start 121.125 88.265) (end 122.555 88.265) (width 0.254) (layer F.Cu) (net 1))
 (segment (start 123.825 89.535) (end 126.525 89.535) (width 0.254) (layer F.Cu) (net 1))
 (segment (start 122.555 88.265) (end 123.825 89.535) (width 0.254) (layer F.Cu) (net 1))
 (segment (start 132.08 94.06) (end 132.08 97.695) (width 0.254) (layer F.Cu) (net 1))
 (segment (start 123.825 93.98) (end 123.825 98.425) (width 0.254) (layer B.Cu) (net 2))
 (via (at 123.825 98.425) (size 0.6858) (drill 0.3302) (layers F.Cu B.Cu) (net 2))
 (segment (start 116.205 94.06) (end 116.205 98.595) (width 0.254) (layer F.Cu) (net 3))
 (segment (start 121.125 90.805) (end 120.015 90.805) (width 0.254) (layer F.Cu) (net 4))
 (via (at 118.745 92.075) (size 0.6858) (drill 0.3302) (layers F.Cu B.Cu) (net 4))
 (segment (start 120.015 90.805) (end 118.745 92.075) (width 0.254) (layer F.Cu) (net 4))
 (segment (start 126.525 86.995) (end 126.525 85.565) (width 0.254) (layer F.Cu) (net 4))
 (via (at 127 85.09) (size 0.6858) (drill 0.3302) (layers F.Cu B.Cu) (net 4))
 (segment (start 126.525 85.565) (end 127 85.09) (width 0.254) (layer F.Cu) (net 4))
 (segment (start 126.525 86.995) (end 128.905 86.995) (width 0.254) (layer F.Cu) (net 4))
 (segment (start 130.89 85.01) (end 132.08 85.01) (width 0.254) (layer F.Cu) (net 4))
 (segment (start 128.905 86.995) (end 130.89 85.01) (width 0.254) (layer F.Cu) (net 4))
 (segment (start 126.525 88.265) (end 129.54 88.265) (width 0.254) (layer F.Cu) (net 5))
 (segment (start 130.095 87.71) (end 132.08 87.71) (width 0.254) (layer F.Cu) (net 5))
 (segment (start 129.54 88.265) (end 130.095 87.71) (width 0.254) (layer F.Cu) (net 5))
 (segment (start 132.08 87.71) (end 132.08 91.36) (width 0.254) (layer F.Cu) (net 5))
 (segment (start 121.125 89.535) (end 118.03 89.535) (width 0.254) (layer F.Cu) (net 6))
 (segment (start 118.03 89.535) (end 116.205 91.36) (width 0.254) (layer F.Cu) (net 6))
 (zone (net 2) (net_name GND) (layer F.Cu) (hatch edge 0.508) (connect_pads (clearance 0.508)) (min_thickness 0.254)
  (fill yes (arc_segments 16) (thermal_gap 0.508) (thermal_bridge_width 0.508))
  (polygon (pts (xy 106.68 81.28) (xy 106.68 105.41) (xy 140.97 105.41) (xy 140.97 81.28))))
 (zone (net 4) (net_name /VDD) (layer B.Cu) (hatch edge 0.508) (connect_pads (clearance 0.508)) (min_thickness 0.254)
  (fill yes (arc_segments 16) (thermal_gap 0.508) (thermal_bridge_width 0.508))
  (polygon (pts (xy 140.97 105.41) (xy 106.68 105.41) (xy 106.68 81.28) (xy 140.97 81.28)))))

